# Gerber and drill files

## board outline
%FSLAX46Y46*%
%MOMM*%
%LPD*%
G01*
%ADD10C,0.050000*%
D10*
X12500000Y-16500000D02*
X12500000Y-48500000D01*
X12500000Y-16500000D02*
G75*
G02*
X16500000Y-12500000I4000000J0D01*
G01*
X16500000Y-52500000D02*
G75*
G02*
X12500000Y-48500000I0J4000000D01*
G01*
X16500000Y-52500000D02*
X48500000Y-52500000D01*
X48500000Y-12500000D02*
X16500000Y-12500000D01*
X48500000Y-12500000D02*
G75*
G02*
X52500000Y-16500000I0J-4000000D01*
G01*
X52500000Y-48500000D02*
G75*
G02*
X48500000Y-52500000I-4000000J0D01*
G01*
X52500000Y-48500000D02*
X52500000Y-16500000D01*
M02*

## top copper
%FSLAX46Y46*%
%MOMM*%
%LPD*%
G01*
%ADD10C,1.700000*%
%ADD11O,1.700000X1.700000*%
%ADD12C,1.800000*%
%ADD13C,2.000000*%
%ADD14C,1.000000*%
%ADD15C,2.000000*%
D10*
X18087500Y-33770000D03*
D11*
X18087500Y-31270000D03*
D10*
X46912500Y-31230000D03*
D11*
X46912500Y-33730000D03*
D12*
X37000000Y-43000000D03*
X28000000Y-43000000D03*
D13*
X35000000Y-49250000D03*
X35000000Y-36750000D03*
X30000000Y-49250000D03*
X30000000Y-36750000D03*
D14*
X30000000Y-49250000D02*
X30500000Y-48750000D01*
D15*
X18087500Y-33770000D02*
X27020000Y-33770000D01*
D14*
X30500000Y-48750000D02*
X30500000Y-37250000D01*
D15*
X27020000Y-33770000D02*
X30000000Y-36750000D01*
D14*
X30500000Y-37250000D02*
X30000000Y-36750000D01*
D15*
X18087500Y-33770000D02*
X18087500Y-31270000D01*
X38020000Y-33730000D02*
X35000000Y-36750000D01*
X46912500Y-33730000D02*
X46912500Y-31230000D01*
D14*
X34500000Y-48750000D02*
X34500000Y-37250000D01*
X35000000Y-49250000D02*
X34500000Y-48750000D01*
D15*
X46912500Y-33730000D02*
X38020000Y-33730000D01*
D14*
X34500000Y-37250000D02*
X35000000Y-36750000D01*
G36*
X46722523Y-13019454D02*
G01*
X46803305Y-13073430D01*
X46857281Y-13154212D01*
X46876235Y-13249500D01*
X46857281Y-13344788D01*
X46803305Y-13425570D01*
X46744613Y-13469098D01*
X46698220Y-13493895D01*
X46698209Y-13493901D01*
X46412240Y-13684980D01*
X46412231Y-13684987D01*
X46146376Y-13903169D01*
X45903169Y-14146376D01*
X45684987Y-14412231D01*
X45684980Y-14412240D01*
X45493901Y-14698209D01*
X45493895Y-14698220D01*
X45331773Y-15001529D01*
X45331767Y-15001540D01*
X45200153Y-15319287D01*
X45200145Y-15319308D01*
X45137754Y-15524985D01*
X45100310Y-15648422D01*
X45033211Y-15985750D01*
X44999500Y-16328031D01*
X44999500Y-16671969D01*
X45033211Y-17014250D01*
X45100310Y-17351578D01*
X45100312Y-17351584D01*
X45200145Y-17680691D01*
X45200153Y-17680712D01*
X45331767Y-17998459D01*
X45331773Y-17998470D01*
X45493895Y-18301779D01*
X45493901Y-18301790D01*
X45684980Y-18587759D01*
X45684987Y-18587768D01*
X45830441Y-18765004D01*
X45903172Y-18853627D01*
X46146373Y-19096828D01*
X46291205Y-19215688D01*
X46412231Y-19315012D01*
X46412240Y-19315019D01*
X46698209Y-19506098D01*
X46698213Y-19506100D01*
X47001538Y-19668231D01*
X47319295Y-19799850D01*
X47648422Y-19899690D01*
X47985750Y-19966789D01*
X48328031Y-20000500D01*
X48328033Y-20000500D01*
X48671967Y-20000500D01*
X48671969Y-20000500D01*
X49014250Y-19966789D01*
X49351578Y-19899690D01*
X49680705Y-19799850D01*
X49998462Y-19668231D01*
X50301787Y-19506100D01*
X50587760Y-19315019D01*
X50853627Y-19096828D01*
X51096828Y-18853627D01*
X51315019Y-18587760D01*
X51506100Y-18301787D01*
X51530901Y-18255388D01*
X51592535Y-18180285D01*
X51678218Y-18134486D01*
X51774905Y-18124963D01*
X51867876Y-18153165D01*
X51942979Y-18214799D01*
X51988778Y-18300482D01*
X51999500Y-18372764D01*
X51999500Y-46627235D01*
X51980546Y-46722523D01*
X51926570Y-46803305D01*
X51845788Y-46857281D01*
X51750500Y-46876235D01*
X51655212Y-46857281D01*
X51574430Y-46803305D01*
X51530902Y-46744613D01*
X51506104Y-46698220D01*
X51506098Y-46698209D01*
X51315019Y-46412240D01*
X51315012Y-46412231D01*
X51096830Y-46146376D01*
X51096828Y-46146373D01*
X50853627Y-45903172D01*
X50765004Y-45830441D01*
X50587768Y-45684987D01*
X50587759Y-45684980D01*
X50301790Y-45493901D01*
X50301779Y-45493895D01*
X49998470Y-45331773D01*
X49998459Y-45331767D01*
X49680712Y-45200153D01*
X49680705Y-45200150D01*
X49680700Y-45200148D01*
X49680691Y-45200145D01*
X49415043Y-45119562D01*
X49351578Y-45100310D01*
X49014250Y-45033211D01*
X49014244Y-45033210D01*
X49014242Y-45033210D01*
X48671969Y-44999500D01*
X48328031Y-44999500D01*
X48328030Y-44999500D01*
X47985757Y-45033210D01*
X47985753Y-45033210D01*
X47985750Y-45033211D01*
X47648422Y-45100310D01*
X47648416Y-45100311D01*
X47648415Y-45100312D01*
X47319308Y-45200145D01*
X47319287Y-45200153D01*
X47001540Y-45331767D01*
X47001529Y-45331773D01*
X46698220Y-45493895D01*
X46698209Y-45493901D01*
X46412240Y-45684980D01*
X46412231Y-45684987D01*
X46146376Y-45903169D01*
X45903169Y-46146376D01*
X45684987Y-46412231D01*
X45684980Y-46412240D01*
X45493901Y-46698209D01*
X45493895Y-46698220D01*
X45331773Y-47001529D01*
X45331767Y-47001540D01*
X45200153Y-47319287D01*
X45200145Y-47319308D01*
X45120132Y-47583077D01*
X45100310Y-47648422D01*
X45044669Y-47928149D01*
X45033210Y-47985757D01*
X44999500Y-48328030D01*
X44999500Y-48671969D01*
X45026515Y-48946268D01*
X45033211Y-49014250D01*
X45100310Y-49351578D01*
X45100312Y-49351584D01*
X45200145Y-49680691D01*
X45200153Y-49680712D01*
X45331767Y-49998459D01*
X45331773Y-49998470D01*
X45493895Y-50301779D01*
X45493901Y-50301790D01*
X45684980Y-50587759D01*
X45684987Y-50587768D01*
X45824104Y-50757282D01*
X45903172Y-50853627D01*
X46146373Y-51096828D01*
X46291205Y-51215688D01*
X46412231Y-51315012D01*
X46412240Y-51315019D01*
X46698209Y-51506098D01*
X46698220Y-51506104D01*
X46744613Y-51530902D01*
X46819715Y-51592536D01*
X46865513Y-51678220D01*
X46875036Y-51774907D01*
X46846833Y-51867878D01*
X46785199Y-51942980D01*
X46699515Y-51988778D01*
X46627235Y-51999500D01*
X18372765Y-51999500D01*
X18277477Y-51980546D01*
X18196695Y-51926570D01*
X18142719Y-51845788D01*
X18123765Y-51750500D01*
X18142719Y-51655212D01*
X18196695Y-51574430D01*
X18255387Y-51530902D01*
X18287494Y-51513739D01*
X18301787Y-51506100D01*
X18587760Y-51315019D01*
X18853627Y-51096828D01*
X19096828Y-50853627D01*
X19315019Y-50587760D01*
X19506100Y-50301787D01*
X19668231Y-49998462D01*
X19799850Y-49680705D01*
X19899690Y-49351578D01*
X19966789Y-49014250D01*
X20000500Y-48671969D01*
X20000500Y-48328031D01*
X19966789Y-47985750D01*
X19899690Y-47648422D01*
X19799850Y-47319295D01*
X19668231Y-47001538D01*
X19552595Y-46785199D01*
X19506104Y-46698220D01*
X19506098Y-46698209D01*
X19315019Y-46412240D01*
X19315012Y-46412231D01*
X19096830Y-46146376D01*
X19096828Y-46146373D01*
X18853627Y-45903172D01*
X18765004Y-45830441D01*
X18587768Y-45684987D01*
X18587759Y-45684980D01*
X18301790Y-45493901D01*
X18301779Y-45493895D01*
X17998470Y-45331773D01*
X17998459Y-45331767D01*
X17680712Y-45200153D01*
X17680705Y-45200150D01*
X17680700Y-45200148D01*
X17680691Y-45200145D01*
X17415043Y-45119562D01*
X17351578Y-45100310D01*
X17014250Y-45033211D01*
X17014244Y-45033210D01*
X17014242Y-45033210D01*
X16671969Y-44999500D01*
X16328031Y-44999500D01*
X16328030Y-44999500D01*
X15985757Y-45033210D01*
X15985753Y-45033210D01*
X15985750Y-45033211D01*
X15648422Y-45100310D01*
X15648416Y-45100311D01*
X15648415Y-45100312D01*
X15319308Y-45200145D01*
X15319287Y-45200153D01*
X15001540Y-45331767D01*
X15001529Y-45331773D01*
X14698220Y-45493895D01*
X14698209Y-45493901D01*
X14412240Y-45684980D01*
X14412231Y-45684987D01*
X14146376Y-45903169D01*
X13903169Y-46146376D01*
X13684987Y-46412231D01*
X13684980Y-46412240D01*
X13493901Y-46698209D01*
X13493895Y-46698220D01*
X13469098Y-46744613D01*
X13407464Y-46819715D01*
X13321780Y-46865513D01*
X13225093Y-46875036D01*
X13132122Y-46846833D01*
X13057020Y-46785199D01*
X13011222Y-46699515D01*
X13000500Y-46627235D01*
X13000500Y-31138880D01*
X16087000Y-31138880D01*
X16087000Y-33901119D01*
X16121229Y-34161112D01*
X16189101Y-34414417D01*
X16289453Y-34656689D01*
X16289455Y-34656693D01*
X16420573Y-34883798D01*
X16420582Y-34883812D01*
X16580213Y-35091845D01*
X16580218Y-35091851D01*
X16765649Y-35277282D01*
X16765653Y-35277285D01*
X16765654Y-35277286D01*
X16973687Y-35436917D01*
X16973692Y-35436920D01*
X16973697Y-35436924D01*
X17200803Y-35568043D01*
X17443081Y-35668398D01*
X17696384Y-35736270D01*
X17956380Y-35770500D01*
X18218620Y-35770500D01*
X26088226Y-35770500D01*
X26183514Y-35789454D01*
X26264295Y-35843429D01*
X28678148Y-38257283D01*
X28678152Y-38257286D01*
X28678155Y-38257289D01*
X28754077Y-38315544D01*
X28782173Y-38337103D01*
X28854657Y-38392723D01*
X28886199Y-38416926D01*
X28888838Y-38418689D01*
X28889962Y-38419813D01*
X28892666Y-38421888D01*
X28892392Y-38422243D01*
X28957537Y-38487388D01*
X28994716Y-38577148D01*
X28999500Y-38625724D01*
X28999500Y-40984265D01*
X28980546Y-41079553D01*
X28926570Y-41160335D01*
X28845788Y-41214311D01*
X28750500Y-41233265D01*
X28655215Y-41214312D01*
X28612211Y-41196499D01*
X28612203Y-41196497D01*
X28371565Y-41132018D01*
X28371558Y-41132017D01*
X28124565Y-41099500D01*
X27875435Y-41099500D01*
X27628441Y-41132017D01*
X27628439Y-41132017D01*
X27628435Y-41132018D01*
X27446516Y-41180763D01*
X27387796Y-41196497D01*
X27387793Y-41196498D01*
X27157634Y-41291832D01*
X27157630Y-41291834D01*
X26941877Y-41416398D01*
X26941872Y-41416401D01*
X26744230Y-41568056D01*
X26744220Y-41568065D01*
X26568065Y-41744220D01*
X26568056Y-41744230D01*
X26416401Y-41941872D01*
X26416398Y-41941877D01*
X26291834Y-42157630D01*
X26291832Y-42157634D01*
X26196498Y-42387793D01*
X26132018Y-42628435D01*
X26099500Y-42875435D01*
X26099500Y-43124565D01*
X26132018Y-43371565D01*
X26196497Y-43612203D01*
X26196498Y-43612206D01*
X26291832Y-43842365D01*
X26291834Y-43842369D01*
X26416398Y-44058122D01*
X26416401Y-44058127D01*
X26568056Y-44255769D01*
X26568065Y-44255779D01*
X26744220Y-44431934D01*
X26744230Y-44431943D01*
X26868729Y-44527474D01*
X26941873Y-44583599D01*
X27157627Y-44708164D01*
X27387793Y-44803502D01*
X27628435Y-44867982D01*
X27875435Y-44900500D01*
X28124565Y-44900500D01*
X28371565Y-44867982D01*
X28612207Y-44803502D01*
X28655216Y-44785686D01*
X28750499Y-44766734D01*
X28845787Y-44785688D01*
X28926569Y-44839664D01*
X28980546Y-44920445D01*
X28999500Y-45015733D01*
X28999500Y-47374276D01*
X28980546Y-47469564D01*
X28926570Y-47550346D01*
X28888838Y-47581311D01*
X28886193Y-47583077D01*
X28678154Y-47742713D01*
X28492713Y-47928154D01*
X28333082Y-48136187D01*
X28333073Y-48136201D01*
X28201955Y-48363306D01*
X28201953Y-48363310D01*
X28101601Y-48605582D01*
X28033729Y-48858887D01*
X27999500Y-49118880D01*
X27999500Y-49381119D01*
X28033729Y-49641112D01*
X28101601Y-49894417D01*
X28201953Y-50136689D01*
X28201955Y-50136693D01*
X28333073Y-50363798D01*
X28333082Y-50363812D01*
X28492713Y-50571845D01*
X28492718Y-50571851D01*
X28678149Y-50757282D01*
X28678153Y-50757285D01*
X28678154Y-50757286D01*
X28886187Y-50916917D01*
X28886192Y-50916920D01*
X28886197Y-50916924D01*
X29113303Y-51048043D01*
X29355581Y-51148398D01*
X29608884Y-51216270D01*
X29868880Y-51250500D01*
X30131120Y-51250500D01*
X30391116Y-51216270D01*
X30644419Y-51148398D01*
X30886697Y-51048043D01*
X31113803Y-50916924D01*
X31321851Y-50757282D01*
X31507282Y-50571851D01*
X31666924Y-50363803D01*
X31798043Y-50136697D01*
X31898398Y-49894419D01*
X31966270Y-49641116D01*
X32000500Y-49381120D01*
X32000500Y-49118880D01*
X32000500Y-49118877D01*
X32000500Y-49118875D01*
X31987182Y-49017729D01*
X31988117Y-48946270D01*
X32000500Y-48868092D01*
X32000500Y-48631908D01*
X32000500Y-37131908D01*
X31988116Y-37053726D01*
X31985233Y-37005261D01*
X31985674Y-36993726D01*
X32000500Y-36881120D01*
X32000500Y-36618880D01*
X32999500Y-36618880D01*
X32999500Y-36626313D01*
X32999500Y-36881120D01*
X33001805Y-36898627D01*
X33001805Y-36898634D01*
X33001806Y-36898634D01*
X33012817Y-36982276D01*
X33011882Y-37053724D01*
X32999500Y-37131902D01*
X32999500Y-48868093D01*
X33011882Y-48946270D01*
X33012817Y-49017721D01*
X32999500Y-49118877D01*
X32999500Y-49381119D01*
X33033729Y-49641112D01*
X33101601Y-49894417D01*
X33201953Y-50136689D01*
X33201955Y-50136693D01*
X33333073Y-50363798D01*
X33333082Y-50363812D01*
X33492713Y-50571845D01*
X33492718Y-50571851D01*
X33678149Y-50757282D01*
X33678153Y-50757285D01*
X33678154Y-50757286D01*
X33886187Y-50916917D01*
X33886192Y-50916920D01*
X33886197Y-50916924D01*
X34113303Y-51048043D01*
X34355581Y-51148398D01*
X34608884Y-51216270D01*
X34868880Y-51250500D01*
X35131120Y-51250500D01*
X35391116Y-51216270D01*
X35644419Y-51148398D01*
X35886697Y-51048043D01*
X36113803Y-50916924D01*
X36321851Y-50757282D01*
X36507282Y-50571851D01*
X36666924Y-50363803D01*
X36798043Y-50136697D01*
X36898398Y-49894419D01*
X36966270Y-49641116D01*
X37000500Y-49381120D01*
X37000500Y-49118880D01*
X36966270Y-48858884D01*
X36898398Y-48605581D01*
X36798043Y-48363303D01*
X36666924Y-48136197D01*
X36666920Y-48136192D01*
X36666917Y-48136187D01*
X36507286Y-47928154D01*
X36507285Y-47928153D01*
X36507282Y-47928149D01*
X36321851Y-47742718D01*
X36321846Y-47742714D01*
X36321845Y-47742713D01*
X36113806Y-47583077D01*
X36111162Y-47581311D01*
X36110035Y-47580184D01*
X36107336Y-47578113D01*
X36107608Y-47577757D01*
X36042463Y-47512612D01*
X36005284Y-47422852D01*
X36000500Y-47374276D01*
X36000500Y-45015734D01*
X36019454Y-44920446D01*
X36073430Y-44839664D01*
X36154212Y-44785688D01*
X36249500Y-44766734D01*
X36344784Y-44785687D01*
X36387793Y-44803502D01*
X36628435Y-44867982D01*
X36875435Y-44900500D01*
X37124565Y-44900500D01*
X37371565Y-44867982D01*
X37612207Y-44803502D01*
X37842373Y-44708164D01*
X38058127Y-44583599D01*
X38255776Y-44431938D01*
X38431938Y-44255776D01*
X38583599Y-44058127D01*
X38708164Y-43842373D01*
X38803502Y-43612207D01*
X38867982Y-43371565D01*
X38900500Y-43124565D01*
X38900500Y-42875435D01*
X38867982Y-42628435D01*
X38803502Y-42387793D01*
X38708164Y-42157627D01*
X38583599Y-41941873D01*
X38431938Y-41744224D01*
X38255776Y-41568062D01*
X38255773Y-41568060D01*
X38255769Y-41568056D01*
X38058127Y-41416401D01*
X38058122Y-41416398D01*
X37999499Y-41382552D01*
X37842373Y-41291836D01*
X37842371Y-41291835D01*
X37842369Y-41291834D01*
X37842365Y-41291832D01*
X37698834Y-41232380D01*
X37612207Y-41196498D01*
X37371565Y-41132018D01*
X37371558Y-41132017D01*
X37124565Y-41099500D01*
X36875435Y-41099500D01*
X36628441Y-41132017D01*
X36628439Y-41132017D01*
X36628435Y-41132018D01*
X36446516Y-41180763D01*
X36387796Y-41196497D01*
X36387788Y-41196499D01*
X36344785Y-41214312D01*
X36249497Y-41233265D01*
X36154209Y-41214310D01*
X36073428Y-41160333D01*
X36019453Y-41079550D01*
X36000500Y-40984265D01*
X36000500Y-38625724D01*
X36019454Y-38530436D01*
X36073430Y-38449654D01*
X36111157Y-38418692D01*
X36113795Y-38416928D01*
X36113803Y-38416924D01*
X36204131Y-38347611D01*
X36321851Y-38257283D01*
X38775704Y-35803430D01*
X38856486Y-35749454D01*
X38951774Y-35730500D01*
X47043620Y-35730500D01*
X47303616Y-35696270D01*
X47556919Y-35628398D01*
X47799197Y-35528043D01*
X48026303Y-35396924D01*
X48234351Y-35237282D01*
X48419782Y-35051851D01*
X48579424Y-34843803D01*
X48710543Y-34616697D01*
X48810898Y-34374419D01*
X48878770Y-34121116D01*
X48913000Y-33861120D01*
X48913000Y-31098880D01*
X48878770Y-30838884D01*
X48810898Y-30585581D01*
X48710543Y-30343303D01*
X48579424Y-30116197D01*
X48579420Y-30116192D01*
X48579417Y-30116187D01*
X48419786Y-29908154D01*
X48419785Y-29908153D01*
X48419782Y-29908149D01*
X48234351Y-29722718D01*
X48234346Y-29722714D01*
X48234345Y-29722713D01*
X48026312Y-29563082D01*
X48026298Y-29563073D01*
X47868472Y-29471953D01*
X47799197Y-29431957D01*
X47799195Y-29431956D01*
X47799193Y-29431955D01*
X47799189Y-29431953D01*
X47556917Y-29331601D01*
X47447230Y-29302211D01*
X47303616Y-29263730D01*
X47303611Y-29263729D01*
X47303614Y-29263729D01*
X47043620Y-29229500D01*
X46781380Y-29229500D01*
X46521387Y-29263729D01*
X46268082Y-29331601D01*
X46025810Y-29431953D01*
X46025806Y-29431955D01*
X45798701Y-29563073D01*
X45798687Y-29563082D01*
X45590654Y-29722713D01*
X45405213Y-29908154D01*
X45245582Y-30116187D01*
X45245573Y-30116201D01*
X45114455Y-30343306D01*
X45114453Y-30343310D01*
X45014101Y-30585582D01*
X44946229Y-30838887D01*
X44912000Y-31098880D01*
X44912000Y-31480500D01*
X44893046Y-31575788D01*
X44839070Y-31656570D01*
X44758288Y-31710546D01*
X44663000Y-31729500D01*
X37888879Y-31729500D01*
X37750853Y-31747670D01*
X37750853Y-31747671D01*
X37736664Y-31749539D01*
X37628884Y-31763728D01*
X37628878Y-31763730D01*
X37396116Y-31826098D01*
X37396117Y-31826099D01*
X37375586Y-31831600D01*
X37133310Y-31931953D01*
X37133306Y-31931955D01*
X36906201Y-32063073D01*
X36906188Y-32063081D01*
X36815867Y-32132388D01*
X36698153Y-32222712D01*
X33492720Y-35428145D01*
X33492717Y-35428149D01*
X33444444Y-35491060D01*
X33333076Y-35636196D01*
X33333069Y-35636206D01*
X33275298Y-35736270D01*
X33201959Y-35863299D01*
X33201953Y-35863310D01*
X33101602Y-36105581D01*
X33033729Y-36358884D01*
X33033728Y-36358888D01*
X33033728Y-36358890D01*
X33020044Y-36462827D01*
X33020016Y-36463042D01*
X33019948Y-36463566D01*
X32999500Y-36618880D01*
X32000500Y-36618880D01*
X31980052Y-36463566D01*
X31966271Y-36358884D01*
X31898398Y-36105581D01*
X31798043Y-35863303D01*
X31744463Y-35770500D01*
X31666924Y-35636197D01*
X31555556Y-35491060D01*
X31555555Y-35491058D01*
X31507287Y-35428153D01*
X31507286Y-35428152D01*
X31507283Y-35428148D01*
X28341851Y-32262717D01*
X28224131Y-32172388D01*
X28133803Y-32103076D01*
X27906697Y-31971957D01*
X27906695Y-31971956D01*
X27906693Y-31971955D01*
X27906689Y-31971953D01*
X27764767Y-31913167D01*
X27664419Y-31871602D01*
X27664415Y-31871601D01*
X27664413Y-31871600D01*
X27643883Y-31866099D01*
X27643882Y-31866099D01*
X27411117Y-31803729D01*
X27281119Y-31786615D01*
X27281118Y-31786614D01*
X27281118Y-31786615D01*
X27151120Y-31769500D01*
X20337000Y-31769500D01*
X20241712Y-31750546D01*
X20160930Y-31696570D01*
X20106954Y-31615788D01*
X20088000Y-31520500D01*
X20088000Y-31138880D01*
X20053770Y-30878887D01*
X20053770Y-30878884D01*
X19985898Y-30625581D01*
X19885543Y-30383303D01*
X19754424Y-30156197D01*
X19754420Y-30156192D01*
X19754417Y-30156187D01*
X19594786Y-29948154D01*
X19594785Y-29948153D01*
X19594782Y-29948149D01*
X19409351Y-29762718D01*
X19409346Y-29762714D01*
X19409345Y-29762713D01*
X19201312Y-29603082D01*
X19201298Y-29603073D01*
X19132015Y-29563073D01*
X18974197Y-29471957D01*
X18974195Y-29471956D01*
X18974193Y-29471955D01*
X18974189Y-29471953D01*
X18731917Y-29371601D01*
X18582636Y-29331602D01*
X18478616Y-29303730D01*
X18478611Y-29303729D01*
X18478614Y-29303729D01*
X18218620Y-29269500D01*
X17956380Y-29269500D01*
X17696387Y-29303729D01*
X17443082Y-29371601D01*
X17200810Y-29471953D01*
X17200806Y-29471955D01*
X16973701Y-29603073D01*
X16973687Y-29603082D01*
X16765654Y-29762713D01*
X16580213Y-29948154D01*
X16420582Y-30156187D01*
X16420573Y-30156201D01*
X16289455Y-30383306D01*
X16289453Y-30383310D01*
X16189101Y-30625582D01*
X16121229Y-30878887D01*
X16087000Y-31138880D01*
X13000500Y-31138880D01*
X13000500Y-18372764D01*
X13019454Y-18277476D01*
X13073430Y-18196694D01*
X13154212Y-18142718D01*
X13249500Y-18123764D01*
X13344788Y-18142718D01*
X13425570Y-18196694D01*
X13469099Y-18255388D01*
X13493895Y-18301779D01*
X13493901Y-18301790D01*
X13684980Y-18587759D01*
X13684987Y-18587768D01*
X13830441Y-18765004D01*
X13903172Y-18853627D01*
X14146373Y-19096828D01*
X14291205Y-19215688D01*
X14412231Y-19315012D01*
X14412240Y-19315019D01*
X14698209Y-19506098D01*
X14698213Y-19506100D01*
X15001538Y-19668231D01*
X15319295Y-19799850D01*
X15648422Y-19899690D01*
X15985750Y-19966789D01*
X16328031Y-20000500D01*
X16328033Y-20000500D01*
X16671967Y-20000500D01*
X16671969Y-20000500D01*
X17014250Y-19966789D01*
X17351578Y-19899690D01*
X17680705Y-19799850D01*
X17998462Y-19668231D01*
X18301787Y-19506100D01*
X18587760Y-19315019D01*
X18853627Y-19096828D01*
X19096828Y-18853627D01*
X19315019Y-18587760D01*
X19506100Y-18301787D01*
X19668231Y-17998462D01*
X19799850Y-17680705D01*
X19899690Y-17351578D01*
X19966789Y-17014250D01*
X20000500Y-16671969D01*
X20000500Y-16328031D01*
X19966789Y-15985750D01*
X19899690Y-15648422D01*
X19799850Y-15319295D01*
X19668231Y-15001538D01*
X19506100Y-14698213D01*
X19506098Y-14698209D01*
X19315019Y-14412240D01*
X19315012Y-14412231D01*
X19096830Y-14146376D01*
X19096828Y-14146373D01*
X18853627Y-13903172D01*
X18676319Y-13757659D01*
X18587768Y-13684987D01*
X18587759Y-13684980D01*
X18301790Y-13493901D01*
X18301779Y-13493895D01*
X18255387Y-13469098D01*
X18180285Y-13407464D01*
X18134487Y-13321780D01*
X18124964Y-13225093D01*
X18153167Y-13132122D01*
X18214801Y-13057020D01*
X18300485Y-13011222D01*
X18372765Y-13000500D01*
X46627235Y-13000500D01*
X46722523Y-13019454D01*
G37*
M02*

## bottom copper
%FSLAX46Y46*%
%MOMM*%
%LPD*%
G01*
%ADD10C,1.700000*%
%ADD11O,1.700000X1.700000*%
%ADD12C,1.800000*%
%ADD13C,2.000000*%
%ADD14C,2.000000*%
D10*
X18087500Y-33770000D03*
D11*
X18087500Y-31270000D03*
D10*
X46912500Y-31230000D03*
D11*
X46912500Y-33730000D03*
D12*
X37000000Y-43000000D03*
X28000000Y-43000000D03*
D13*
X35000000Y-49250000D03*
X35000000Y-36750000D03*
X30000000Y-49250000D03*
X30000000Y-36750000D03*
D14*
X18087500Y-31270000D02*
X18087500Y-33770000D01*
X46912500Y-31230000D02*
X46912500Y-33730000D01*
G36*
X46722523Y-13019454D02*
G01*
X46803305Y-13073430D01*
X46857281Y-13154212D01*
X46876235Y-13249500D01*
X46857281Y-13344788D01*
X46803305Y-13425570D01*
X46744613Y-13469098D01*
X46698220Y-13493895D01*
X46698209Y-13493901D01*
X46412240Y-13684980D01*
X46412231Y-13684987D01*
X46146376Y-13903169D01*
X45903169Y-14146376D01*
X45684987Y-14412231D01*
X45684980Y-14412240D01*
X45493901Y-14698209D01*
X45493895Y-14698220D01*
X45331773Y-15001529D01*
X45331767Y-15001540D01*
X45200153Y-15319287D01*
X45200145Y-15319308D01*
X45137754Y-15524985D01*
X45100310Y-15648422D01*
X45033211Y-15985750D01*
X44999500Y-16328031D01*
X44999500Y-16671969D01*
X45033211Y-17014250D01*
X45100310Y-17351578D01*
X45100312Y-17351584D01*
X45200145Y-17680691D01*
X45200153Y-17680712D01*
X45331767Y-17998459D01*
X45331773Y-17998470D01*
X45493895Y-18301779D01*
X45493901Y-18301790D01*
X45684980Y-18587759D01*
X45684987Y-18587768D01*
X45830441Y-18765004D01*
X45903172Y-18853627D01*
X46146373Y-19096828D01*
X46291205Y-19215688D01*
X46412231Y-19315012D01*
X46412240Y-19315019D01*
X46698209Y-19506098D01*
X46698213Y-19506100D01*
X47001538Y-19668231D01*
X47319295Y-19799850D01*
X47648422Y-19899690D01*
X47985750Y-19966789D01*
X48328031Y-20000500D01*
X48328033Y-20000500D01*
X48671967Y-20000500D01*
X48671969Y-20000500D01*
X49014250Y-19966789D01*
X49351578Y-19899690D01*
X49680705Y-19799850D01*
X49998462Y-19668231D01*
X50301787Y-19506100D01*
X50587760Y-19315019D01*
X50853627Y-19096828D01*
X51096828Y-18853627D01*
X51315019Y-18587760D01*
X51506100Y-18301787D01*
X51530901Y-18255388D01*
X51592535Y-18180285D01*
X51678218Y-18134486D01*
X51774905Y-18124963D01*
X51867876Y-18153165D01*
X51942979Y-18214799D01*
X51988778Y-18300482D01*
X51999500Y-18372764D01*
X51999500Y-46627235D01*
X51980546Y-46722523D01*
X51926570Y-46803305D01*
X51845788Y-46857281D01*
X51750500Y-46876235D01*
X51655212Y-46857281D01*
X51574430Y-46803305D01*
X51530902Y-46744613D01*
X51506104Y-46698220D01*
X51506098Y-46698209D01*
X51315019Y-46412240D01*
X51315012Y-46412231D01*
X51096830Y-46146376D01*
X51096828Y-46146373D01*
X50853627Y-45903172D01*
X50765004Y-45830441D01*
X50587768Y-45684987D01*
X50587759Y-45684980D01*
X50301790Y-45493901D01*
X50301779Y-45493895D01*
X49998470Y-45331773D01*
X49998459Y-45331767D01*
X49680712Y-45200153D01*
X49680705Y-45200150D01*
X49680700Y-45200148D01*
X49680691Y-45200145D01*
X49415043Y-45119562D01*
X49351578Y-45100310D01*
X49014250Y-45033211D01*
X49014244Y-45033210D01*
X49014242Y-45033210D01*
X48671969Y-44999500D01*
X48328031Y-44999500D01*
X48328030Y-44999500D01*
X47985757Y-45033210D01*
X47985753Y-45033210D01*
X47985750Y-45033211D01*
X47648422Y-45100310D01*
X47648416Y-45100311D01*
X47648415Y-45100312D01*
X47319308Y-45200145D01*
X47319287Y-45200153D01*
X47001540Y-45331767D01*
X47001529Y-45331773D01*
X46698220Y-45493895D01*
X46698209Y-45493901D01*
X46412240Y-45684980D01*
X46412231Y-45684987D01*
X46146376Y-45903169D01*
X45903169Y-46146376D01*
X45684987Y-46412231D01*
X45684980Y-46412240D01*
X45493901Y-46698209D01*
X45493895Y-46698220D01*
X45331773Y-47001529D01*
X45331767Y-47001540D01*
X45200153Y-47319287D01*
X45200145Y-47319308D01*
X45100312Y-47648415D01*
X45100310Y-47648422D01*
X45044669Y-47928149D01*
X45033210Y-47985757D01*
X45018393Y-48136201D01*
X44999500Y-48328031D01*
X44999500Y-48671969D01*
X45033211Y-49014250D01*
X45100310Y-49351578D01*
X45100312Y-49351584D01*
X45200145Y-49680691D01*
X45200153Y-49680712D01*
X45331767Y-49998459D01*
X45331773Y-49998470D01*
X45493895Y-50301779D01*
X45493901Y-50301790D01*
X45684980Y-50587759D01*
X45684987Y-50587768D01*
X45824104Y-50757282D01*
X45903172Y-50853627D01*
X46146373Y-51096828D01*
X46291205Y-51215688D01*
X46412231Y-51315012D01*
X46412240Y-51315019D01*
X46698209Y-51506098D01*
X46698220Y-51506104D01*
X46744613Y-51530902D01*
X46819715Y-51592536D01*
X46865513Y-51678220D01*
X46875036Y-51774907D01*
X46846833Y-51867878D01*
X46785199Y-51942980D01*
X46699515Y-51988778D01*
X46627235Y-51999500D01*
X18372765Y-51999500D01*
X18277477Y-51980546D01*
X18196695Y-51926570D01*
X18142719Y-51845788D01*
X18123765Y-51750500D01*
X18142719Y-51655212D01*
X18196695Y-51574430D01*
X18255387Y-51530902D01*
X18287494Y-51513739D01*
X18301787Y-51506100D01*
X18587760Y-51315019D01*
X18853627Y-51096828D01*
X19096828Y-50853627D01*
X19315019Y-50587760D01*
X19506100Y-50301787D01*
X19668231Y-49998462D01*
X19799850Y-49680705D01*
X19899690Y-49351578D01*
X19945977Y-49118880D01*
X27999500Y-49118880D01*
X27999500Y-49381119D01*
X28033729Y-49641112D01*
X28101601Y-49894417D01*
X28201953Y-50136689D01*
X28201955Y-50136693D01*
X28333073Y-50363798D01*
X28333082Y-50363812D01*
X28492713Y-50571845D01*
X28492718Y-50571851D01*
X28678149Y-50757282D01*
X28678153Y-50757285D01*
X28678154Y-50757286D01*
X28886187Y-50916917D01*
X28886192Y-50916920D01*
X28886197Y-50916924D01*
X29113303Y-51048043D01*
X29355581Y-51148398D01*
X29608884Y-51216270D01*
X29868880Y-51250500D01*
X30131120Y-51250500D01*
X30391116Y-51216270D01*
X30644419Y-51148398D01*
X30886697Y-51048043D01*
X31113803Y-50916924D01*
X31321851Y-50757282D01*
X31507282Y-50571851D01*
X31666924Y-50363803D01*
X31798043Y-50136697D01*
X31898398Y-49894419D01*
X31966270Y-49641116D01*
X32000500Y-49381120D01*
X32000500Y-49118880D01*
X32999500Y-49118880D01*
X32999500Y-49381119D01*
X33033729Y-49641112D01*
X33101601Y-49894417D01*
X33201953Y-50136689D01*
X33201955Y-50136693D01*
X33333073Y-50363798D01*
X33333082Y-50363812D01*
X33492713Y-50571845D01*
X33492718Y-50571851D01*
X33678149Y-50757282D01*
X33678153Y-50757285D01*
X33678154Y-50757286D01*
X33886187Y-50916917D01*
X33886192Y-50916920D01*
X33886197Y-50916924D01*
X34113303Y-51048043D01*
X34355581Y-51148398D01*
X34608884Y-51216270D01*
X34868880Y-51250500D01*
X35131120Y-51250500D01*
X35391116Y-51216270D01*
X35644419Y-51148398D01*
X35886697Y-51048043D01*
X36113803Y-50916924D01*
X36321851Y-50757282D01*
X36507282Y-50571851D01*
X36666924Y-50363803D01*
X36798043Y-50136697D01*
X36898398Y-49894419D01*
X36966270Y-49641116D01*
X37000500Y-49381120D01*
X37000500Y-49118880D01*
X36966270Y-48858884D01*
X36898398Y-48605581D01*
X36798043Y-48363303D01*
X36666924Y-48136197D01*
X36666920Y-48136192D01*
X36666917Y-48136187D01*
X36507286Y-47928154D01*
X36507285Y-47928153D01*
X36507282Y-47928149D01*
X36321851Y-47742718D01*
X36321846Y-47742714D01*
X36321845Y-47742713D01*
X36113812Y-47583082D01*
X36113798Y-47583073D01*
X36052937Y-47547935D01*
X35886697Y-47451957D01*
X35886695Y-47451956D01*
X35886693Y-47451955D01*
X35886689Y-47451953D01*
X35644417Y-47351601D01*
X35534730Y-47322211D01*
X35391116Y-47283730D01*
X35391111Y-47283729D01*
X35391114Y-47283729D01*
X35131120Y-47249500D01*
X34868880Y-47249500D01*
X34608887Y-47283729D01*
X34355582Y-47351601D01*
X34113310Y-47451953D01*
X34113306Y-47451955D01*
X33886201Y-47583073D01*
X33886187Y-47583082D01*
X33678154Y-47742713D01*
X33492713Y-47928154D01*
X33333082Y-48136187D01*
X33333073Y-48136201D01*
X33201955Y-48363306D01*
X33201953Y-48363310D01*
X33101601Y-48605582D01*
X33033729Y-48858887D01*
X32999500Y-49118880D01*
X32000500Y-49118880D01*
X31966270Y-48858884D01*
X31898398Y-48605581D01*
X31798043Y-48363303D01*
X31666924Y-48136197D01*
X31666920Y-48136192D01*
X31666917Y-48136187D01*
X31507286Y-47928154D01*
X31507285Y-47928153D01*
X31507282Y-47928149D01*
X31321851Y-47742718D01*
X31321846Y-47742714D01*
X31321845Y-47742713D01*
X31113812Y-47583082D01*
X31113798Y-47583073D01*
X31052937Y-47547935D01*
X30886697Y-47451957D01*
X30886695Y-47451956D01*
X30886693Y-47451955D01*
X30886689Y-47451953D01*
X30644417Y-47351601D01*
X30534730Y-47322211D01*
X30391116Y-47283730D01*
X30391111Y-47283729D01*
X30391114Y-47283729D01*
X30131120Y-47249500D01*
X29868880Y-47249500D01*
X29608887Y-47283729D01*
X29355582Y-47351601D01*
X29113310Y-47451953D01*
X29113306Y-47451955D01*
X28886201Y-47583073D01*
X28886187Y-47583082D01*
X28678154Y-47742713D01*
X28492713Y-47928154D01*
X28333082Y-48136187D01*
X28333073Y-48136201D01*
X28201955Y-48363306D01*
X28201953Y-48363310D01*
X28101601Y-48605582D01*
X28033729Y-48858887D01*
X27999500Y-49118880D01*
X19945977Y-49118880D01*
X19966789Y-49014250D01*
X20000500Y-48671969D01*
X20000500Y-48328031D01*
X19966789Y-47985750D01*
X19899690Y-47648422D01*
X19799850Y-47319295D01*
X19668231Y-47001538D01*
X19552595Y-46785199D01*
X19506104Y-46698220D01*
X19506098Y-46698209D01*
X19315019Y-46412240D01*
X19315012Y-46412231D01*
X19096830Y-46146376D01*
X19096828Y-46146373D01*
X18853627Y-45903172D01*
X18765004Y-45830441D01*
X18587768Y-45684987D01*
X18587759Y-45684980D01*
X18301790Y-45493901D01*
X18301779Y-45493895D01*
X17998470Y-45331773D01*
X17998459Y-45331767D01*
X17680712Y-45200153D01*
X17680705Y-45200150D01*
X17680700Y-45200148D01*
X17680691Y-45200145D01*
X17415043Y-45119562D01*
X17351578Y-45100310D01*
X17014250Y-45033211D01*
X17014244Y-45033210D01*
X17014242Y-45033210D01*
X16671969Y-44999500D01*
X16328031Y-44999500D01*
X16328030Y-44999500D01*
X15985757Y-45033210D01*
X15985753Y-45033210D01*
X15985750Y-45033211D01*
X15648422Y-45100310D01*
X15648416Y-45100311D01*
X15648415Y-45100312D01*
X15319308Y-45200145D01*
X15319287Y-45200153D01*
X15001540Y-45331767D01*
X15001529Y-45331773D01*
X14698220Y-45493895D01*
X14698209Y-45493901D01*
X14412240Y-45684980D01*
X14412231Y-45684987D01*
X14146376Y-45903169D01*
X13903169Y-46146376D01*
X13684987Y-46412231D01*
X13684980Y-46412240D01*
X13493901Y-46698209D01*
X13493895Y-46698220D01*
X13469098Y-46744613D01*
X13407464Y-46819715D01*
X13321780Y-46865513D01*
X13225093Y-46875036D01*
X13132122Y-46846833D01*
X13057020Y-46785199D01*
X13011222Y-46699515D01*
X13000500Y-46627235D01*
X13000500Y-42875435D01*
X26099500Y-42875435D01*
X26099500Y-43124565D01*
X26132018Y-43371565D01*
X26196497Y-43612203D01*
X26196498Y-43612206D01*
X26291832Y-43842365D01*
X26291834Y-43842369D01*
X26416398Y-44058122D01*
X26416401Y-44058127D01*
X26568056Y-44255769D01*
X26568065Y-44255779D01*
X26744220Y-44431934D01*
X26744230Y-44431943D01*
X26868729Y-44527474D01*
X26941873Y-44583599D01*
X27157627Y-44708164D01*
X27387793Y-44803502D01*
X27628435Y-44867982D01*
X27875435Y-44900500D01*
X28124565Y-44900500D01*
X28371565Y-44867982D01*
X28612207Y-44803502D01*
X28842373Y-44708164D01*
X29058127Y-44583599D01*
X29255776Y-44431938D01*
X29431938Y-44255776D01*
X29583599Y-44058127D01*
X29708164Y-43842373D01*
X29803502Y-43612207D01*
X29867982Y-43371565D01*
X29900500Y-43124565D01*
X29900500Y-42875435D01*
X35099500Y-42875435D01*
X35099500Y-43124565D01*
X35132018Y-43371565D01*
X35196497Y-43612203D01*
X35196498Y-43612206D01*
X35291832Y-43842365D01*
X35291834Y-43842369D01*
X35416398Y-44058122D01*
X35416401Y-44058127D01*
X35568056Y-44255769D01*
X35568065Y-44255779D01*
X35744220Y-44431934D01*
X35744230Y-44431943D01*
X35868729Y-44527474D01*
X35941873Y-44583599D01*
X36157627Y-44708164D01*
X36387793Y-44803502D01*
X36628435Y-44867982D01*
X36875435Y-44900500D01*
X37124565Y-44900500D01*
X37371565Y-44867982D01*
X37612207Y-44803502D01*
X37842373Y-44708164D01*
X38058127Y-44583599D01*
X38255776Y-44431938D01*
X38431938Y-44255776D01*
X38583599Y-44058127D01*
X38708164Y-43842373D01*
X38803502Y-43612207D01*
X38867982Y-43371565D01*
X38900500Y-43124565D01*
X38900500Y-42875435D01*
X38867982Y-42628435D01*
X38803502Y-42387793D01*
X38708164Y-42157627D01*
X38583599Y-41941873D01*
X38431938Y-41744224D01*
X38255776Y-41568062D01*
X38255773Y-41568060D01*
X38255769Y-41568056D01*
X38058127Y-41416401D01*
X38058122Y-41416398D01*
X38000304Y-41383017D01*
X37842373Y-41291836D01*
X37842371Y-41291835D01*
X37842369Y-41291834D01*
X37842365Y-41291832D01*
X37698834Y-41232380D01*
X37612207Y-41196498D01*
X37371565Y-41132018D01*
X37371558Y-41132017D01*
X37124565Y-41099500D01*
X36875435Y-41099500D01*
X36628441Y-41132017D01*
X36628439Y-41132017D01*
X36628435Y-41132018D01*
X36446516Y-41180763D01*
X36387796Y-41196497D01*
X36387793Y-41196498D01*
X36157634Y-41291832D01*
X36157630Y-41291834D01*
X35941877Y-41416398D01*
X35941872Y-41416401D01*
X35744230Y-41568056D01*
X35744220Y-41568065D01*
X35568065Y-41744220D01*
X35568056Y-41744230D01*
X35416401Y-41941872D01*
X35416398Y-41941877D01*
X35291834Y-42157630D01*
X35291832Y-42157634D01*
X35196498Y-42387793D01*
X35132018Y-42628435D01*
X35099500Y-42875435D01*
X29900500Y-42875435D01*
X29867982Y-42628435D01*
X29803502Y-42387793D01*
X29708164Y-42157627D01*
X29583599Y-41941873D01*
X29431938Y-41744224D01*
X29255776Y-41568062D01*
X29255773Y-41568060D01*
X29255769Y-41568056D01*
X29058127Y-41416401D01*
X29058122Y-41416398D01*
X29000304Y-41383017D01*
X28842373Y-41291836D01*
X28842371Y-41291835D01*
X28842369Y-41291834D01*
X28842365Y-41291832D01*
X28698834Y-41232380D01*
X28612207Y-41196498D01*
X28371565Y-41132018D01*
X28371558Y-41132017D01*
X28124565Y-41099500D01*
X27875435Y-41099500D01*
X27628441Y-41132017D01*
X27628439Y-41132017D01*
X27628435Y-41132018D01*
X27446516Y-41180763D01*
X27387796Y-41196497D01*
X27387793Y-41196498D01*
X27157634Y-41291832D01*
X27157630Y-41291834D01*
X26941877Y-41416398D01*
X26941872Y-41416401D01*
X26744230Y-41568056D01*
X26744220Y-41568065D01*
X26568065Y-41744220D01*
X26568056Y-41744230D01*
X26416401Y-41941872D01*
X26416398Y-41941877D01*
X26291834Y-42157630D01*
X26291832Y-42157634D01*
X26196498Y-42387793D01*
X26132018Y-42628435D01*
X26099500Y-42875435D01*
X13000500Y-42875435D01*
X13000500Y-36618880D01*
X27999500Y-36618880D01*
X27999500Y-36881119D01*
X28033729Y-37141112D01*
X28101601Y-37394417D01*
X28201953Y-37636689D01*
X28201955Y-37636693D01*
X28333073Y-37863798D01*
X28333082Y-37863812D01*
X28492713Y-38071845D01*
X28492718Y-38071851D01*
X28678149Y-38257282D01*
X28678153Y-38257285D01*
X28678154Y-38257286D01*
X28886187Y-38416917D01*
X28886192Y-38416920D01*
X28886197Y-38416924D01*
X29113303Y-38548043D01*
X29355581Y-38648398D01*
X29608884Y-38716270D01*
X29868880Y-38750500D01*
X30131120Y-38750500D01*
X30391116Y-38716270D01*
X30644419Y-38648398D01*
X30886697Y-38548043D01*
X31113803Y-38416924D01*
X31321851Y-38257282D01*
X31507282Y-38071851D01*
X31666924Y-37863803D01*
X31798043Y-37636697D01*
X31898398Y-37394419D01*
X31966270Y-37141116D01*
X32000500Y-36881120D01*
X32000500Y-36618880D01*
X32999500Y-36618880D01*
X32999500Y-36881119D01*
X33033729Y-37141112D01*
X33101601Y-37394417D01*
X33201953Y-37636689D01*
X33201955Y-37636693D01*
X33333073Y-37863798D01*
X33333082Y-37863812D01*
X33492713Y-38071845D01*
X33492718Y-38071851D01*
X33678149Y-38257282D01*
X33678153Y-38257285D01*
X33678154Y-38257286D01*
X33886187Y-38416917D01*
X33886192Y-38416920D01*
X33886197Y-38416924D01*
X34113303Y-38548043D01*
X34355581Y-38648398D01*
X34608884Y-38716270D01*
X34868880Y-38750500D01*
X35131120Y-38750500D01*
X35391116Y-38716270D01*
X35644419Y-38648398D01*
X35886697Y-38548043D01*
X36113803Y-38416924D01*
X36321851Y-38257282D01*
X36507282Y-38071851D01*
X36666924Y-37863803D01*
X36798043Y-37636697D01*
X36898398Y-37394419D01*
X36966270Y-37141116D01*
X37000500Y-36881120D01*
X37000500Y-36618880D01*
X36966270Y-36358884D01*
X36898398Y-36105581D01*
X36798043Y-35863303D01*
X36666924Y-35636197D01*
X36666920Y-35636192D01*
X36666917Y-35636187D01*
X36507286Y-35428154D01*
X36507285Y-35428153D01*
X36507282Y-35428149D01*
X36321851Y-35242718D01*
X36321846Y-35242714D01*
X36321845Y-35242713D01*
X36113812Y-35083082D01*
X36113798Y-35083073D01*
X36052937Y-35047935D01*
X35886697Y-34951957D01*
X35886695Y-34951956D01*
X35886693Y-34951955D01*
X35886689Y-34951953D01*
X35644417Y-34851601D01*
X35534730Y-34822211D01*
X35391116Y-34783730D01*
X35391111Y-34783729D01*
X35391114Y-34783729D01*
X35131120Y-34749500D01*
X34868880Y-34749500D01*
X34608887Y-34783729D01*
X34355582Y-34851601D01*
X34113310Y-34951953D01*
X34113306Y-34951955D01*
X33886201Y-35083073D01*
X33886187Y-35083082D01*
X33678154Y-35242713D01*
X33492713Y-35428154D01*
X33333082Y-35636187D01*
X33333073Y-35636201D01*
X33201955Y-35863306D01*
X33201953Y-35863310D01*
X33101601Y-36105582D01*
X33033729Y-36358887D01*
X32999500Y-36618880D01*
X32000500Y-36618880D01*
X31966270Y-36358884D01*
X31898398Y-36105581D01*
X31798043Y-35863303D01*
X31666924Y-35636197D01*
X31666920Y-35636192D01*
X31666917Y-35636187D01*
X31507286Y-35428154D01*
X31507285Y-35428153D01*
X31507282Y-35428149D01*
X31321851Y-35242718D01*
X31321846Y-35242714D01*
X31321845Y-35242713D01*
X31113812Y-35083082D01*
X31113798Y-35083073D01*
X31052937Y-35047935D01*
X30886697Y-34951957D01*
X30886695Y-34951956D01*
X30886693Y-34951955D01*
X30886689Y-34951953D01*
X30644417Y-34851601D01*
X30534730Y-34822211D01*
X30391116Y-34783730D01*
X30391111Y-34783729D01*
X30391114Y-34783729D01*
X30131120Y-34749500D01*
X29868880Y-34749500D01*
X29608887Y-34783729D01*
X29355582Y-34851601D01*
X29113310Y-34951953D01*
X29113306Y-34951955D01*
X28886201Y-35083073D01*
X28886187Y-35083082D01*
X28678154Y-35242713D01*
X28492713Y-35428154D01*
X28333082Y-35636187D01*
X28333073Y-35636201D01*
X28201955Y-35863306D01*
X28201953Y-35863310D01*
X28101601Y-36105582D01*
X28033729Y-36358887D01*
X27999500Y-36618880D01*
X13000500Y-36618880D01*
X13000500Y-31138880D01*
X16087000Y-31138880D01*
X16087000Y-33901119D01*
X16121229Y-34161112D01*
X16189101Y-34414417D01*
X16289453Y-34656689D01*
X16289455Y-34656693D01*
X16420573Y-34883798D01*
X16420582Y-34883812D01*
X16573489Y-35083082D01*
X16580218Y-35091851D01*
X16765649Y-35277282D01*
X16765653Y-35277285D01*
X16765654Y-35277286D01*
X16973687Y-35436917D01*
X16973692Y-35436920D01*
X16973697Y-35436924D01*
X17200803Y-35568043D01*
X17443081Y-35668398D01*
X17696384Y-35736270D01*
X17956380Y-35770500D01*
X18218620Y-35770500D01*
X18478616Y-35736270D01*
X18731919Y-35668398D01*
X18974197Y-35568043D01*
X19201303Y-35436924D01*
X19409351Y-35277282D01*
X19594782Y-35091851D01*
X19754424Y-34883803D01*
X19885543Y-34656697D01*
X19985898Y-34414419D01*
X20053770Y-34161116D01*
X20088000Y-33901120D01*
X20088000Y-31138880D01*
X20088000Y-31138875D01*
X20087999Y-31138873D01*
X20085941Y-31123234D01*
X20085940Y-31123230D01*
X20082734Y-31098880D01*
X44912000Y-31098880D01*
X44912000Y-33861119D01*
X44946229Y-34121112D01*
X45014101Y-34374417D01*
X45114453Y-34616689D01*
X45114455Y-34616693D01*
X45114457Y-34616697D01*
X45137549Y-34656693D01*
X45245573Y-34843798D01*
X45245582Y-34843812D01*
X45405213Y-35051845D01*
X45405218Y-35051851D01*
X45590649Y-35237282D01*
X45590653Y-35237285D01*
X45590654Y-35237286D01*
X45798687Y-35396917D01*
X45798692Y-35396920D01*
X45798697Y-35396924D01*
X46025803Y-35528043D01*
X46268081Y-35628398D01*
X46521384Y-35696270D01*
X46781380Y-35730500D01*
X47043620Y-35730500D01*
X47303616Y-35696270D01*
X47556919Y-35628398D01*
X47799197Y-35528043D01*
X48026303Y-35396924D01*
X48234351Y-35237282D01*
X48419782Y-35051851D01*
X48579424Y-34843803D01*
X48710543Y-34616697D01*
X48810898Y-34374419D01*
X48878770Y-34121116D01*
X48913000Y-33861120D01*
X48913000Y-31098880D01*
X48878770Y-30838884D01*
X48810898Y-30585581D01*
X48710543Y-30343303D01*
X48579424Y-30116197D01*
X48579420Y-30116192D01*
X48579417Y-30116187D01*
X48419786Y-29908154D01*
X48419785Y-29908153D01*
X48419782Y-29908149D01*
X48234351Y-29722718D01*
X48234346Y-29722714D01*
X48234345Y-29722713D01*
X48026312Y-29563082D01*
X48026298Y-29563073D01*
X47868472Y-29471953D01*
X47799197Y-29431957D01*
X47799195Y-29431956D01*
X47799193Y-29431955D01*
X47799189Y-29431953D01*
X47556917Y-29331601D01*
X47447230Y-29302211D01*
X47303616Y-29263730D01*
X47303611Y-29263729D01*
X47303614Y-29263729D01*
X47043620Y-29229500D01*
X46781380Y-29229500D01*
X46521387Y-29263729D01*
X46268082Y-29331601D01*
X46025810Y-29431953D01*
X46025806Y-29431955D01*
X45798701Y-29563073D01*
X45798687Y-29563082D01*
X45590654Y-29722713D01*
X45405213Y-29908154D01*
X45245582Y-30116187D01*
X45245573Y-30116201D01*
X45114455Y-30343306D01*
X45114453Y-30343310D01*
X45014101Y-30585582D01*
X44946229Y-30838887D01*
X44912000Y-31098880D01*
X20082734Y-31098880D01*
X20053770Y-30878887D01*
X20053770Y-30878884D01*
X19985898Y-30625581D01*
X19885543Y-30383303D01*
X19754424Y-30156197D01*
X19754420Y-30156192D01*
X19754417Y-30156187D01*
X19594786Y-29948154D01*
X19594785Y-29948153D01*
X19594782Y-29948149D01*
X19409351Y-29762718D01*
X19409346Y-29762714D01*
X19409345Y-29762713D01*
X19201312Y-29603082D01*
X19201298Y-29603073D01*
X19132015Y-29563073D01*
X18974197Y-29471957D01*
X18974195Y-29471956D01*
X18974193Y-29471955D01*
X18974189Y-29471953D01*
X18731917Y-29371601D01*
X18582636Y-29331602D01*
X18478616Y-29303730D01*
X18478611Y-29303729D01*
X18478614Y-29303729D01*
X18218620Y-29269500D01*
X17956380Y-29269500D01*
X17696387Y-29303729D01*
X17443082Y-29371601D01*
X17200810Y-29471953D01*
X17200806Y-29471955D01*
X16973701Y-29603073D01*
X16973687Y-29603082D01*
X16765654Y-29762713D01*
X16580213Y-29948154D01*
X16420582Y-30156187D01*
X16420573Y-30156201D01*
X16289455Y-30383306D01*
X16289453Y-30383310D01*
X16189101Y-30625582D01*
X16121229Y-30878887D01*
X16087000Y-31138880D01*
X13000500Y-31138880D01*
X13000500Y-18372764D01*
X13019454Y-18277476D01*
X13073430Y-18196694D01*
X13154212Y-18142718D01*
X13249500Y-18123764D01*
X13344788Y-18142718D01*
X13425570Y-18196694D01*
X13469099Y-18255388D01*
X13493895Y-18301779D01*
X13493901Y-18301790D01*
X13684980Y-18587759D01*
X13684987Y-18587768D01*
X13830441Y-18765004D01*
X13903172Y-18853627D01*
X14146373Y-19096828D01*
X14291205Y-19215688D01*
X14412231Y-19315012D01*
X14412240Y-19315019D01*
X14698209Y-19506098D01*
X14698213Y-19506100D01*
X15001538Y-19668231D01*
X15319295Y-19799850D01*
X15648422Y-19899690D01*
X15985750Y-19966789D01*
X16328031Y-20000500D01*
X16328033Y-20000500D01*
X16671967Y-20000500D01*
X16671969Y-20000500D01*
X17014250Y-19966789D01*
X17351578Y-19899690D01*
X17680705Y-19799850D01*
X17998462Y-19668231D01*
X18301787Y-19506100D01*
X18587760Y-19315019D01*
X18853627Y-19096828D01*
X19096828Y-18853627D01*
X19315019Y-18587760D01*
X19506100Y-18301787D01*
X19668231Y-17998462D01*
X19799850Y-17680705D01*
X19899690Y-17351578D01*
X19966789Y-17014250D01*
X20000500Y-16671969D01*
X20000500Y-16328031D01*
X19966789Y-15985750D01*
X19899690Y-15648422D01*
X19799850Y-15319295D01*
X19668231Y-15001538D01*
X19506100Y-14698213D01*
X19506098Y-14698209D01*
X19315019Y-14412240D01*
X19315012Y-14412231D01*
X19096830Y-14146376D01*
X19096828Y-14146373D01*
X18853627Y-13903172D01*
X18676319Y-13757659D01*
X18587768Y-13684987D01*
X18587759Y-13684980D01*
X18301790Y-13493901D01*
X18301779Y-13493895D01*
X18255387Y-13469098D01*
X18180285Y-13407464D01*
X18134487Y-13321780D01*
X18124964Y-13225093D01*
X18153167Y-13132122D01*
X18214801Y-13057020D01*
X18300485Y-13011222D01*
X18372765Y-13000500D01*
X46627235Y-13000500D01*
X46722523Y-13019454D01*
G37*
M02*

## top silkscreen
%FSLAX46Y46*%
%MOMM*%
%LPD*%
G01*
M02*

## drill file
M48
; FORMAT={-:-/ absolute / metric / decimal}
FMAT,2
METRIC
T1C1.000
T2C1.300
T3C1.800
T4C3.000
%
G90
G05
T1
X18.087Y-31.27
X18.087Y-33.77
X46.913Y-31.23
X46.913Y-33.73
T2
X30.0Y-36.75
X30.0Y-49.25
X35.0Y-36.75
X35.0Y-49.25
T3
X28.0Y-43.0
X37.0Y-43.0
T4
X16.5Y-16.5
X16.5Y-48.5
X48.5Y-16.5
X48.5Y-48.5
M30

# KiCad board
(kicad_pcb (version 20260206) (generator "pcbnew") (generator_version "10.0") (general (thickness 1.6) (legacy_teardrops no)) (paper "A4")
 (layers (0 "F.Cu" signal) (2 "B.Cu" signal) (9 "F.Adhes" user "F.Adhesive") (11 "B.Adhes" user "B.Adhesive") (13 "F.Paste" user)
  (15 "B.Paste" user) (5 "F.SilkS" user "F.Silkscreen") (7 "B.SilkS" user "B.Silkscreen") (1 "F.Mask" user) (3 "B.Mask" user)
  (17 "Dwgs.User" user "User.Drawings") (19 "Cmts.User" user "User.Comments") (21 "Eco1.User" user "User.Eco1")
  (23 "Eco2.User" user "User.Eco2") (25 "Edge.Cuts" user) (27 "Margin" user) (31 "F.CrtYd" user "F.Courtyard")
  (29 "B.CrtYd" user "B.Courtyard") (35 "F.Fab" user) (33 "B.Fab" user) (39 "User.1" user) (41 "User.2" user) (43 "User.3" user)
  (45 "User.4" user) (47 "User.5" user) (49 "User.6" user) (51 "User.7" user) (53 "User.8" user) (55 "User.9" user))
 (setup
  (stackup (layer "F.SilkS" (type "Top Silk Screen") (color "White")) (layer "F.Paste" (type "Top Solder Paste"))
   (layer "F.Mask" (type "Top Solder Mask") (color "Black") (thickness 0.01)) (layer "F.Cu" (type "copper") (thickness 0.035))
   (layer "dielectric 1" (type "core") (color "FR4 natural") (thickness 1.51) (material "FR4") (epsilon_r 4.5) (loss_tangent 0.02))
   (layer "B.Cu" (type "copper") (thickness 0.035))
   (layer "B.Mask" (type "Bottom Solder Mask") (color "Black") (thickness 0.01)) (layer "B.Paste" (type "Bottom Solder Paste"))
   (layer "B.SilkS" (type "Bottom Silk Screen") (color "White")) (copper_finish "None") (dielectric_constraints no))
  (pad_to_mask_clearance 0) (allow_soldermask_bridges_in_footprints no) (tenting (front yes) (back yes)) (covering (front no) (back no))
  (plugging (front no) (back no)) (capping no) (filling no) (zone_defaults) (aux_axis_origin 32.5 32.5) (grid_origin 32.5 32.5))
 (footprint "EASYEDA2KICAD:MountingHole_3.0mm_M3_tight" (layer "F.Cu") (at 16.5 16.5 90)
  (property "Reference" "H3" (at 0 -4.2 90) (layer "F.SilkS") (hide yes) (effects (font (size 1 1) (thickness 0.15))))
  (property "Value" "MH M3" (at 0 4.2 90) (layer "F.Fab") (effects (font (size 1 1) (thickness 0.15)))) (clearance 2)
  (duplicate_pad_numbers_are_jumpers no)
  (pad "" np_thru_hole circle (at 0 0 90) (size 3 3) (drill 3) (layers "*.Cu" "*.Mask")))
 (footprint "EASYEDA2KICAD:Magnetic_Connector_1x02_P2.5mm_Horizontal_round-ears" (layer "F.Cu") (at 17.9875 32.5 180)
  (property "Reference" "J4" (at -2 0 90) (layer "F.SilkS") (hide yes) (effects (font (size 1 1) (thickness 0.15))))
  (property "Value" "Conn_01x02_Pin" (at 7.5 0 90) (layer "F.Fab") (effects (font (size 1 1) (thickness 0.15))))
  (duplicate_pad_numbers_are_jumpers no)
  (pad "1" thru_hole circle (at -0.1 -1.27 180) (size 1.7 1.7) (drill 1) (layers "*.Cu" "*.Mask") (remove_unused_layers no)
   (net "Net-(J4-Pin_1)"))
  (pad "2" thru_hole oval (at -0.1 1.23 180) (size 1.7 1.7) (drill 1) (layers "*.Cu" "*.Mask") (remove_unused_layers no)
   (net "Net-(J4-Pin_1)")))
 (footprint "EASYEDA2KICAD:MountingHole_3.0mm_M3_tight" (layer "F.Cu") (at 16.5 48.5 90)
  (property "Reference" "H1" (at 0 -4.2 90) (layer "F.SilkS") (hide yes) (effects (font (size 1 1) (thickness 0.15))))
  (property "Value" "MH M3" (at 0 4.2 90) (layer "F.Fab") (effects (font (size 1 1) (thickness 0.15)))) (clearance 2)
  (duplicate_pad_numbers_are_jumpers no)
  (pad "" np_thru_hole circle (at 0 0 90) (size 3 3) (drill 3) (layers "*.Cu" "*.Mask")))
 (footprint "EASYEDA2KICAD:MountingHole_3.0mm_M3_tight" (layer "F.Cu") (at 48.5 16.5 90)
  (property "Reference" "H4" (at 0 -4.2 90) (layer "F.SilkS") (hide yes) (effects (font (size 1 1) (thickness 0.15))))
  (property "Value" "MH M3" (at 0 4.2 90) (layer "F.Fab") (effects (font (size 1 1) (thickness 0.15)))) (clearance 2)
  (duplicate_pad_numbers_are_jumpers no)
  (pad "" np_thru_hole circle (at 0 0 90) (size 3 3) (drill 3) (layers "*.Cu" "*.Mask")))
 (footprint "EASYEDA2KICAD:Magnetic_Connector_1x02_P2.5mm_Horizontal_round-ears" (layer "F.Cu") (at 47.0125 32.5)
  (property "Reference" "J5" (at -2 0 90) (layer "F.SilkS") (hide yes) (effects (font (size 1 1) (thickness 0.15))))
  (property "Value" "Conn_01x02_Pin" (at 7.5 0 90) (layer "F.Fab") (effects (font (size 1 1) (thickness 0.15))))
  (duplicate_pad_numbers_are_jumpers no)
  (pad "1" thru_hole circle (at -0.1 -1.27) (size 1.7 1.7) (drill 1) (layers "*.Cu" "*.Mask") (remove_unused_layers no)
   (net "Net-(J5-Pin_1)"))
  (pad "2" thru_hole oval (at -0.1 1.23) (size 1.7 1.7) (drill 1) (layers "*.Cu" "*.Mask") (remove_unused_layers no) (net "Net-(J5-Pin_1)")))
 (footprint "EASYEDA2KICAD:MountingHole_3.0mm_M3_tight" (layer "F.Cu") (at 48.5 48.5 90)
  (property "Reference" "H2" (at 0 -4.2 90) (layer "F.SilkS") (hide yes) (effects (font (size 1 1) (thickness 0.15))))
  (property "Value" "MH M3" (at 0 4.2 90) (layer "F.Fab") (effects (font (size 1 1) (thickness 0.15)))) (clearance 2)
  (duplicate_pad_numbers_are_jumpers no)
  (pad "" np_thru_hole circle (at 0 0 90) (size 3 3) (drill 3) (layers "*.Cu" "*.Mask")))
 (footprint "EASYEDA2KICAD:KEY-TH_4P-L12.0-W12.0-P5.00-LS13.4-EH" (layer "B.Cu") (at 32.5 43 -90)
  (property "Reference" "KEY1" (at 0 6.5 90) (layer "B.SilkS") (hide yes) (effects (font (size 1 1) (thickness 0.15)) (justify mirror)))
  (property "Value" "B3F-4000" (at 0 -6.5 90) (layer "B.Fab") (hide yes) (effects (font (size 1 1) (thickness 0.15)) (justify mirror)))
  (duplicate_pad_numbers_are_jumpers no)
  (pad "" thru_hole circle (at 0 -4.5 270) (size 1.8 1.8) (drill 1.8) (layers "*.Cu" "*.Mask") (remove_unused_layers no))
  (pad "" thru_hole circle (at 0 4.5 270) (size 1.8 1.8) (drill 1.8) (layers "*.Cu" "*.Mask") (remove_unused_layers no))
  (pad "1" thru_hole circle (at 6.25 -2.5 270) (size 2 2) (drill 1.300023) (layers "*.Cu" "*.Mask") (remove_unused_layers no)
   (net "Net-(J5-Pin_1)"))
  (pad "2" thru_hole circle (at -6.25 -2.5 270) (size 2 2) (drill 1.300023) (layers "*.Cu" "*.Mask") (remove_unused_layers no)
   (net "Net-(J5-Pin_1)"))
  (pad "3" thru_hole circle (at 6.25 2.5 270) (size 2 2) (drill 1.300023) (layers "*.Cu" "*.Mask") (remove_unused_layers no)
   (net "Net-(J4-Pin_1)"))
  (pad "4" thru_hole circle (at -6.25 2.5 270) (size 2 2) (drill 1.300023) (layers "*.Cu" "*.Mask") (remove_unused_layers no)
   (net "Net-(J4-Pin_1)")))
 (gr_line (start 12.5 16.5) (end 12.5 48.5) (stroke (width 0.05) (type default)) (layer "Edge.Cuts"))
 (gr_arc (start 12.5 16.5) (mid 13.671573 13.671573) (end 16.5 12.5) (stroke (width 0.05) (type default)) (layer "Edge.Cuts"))
 (gr_arc (start 16.5 52.5) (mid 13.671573 51.328427) (end 12.5 48.5) (stroke (width 0.05) (type default)) (layer "Edge.Cuts"))
 (gr_line (start 16.5 52.5) (end 48.5 52.5) (stroke (width 0.05) (type default)) (layer "Edge.Cuts"))
 (gr_line (start 48.5 12.5) (end 16.5 12.5) (stroke (width 0.05) (type default)) (layer "Edge.Cuts"))
 (gr_arc (start 48.5 12.5) (mid 51.328427 13.671573) (end 52.5 16.5) (stroke (width 0.05) (type default)) (layer "Edge.Cuts"))
 (gr_arc (start 52.5 48.5) (mid 51.328427 51.328427) (end 48.5 52.5) (stroke (width 0.05) (type default)) (layer "Edge.Cuts"))
 (gr_line (start 52.5 48.5) (end 52.5 16.5) (stroke (width 0.05) (type default)) (layer "Edge.Cuts"))
 (segment (start 30 49.25) (end 30.5 48.75) (width 1) (layer "F.Cu") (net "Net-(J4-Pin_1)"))
 (segment (start 18.0875 33.77) (end 27.02 33.77) (width 2) (layer "F.Cu") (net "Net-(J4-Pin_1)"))
 (segment (start 30.5 48.75) (end 30.5 37.25) (width 1) (layer "F.Cu") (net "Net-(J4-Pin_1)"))
 (segment (start 27.02 33.77) (end 30 36.75) (width 2) (layer "F.Cu") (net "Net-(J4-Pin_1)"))
 (segment (start 30.5 37.25) (end 30 36.75) (width 1) (layer "F.Cu") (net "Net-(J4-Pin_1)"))
 (segment (start 18.0875 33.77) (end 18.0875 31.27) (width 2) (layer "F.Cu") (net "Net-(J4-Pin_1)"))
 (segment (start 18.0875 31.27) (end 18.0875 33.77) (width 2) (layer "B.Cu") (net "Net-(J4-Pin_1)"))
 (segment (start 38.02 33.73) (end 35 36.75) (width 2) (layer "F.Cu") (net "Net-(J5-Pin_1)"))
 (segment (start 46.9125 33.73) (end 46.9125 31.23) (width 2) (layer "F.Cu") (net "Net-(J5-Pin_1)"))
 (segment (start 34.5 48.75) (end 34.5 37.25) (width 1) (layer "F.Cu") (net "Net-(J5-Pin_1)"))
 (segment (start 35 49.25) (end 34.5 48.75) (width 1) (layer "F.Cu") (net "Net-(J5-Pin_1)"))
 (segment (start 46.9125 33.73) (end 38.02 33.73) (width 2) (layer "F.Cu") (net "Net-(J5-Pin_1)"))
 (segment (start 34.5 37.25) (end 35 36.75) (width 1) (layer "F.Cu") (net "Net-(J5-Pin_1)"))
 (segment (start 46.9125 31.23) (end 46.9125 33.73) (width 2) (layer "B.Cu") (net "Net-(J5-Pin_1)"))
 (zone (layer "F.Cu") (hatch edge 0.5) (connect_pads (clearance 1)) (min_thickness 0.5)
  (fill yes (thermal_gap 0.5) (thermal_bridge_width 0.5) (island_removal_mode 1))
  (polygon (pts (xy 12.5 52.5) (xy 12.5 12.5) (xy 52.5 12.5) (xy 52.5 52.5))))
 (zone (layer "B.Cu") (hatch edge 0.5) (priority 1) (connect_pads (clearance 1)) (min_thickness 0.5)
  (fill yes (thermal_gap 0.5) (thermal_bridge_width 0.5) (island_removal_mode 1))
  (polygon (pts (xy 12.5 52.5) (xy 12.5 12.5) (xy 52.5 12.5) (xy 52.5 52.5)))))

